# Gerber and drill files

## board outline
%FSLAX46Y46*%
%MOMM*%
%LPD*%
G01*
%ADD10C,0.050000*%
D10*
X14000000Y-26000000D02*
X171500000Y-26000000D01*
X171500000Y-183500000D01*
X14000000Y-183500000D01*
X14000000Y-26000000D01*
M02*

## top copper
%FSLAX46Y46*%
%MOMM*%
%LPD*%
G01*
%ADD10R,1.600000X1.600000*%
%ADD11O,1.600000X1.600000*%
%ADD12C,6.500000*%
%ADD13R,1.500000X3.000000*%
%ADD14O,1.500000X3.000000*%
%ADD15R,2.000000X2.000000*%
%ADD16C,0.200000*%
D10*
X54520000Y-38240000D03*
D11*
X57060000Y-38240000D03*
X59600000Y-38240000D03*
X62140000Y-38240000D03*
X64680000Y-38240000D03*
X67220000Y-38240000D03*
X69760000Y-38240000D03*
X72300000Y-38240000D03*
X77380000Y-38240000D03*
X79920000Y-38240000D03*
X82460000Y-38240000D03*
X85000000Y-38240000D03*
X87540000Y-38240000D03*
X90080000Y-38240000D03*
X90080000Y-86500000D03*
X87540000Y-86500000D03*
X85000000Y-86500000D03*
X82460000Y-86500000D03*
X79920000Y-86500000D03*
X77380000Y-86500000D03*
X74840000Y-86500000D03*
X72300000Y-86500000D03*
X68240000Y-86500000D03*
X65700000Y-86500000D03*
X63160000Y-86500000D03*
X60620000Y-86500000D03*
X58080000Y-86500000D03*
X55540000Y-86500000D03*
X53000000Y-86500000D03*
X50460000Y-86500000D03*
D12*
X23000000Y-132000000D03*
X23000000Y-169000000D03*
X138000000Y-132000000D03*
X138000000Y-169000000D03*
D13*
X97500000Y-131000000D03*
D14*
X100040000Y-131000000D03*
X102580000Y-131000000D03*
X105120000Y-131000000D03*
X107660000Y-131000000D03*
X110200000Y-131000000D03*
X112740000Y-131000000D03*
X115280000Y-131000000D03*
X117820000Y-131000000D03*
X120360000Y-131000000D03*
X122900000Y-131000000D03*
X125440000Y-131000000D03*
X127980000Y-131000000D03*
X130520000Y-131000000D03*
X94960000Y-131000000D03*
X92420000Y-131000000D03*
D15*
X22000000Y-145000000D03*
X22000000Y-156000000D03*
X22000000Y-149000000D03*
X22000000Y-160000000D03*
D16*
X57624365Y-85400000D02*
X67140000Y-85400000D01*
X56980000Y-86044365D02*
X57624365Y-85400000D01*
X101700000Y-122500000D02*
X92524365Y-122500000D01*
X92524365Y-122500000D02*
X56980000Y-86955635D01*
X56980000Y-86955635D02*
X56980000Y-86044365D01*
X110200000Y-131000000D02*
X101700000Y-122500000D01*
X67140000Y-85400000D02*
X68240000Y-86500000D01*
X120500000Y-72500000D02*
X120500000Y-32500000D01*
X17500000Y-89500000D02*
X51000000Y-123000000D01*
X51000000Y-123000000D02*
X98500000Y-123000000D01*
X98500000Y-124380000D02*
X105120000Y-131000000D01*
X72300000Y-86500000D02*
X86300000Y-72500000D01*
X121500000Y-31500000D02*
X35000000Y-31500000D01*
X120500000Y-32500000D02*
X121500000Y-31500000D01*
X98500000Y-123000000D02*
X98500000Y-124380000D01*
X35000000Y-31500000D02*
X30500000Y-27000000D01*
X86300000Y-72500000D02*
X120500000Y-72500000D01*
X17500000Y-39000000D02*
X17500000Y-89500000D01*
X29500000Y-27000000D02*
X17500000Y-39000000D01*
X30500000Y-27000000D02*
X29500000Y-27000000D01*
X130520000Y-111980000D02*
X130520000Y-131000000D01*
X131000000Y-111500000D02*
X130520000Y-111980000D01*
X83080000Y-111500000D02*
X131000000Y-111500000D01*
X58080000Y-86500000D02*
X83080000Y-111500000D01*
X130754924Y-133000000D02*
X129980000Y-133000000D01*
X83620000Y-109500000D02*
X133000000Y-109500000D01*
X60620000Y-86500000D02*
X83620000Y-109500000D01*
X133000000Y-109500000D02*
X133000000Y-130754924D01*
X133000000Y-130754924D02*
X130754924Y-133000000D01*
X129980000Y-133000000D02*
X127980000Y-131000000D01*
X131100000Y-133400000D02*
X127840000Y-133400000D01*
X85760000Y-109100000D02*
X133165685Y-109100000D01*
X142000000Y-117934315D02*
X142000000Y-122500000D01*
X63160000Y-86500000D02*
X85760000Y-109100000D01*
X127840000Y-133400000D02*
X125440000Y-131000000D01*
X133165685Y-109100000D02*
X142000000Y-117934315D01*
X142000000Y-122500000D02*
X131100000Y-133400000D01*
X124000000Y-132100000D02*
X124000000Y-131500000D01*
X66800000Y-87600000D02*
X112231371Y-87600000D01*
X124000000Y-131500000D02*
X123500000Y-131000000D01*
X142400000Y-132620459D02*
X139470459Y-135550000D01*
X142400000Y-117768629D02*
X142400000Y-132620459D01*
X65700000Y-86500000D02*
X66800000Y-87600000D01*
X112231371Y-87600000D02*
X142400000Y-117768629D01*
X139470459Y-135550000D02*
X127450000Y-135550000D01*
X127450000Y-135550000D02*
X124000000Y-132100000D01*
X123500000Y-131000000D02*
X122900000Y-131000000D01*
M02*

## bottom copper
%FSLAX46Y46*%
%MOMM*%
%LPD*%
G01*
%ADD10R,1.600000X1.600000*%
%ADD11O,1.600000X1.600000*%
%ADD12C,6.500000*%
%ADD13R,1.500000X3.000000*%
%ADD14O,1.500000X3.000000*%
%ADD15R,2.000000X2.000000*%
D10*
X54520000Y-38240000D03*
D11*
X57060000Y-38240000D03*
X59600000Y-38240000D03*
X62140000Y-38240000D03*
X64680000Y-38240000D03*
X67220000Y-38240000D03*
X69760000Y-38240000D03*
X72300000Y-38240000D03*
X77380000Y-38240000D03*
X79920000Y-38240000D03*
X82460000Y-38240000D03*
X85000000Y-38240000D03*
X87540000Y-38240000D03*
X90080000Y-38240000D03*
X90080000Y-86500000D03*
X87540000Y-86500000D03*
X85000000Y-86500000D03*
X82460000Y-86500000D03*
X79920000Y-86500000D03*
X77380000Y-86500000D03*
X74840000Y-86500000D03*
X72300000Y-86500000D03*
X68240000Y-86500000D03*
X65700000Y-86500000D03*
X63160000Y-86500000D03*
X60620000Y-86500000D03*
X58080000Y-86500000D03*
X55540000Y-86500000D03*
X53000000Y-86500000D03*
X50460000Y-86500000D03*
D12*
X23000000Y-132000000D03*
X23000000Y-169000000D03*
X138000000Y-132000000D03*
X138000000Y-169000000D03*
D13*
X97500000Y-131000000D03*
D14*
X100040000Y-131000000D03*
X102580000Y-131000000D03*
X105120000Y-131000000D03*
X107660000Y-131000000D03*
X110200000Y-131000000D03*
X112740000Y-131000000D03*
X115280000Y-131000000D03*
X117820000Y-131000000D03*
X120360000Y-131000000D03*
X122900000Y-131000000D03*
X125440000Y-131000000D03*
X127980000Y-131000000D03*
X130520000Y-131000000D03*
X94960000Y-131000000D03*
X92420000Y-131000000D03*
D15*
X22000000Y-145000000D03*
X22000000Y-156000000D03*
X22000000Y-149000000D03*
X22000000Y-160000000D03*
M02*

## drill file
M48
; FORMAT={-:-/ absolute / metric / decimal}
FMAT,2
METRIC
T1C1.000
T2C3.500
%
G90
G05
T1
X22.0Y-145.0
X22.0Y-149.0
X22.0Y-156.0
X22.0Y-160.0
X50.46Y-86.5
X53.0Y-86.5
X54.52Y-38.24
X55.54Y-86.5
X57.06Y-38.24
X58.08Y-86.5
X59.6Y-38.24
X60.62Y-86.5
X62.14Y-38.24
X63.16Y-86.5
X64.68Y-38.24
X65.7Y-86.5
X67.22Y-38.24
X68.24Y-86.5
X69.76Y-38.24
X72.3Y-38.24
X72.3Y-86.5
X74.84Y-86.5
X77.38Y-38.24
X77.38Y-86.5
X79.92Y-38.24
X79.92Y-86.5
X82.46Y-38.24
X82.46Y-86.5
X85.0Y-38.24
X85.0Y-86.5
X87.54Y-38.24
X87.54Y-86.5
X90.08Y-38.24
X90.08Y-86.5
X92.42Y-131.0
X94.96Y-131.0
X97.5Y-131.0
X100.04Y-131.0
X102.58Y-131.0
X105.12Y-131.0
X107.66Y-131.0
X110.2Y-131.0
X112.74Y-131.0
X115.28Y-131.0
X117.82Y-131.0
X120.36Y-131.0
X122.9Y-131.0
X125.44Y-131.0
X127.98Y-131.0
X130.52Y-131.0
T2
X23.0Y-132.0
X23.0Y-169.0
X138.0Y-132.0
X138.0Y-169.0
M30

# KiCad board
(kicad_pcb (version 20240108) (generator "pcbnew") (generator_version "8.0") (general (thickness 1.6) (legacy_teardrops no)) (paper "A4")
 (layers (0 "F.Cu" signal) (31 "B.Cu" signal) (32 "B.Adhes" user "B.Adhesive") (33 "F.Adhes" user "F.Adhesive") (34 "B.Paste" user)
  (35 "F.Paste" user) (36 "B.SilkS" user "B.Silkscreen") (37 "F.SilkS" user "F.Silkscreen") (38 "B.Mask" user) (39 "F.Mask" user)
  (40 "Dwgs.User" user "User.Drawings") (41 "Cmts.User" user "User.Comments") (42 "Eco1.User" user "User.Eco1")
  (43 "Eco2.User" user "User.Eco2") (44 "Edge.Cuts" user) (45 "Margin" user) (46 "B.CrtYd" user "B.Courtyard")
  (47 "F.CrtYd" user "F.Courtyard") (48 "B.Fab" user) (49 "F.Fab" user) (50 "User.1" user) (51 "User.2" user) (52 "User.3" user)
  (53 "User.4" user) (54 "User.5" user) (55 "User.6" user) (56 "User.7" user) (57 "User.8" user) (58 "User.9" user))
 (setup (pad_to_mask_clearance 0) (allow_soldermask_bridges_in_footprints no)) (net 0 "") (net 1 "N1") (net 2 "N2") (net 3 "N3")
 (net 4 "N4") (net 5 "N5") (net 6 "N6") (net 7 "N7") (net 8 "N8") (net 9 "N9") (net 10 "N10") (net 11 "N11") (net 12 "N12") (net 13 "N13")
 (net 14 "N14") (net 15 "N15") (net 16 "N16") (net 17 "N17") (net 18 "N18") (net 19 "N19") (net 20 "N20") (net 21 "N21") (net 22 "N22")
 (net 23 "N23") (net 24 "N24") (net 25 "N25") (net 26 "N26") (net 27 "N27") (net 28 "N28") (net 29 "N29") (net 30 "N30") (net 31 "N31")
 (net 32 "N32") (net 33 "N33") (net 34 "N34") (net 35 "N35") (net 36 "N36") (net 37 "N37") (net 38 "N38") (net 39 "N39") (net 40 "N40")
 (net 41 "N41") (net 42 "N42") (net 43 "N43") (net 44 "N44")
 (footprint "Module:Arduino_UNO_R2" (layer "F.Cu") (at 54.52 38.24)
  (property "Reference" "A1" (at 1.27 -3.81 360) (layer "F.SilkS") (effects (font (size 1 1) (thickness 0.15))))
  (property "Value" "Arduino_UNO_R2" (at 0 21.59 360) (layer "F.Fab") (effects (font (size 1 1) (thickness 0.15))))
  (pad "1" thru_hole rect (at 0 0 90) (size 1.6 1.6) (drill 1) (layers "*.Cu" "*.Mask") (remove_unused_layers no) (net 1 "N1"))
  (pad "2" thru_hole oval (at 2.54 0 90) (size 1.6 1.6) (drill 1) (layers "*.Cu" "*.Mask") (remove_unused_layers no) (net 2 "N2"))
  (pad "3" thru_hole oval (at 5.08 0 90) (size 1.6 1.6) (drill 1) (layers "*.Cu" "*.Mask") (remove_unused_layers no) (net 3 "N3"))
  (pad "4" thru_hole oval (at 7.62 0 90) (size 1.6 1.6) (drill 1) (layers "*.Cu" "*.Mask") (remove_unused_layers no) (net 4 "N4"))
  (pad "5" thru_hole oval (at 10.16 0 90) (size 1.6 1.6) (drill 1) (layers "*.Cu" "*.Mask") (remove_unused_layers no) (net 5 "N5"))
  (pad "6" thru_hole oval (at 12.7 0 90) (size 1.6 1.6) (drill 1) (layers "*.Cu" "*.Mask") (remove_unused_layers no) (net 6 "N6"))
  (pad "7" thru_hole oval (at 15.24 0 90) (size 1.6 1.6) (drill 1) (layers "*.Cu" "*.Mask") (remove_unused_layers no) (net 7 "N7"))
  (pad "8" thru_hole oval (at 17.78 0 90) (size 1.6 1.6) (drill 1) (layers "*.Cu" "*.Mask") (remove_unused_layers no) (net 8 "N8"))
  (pad "9" thru_hole oval (at 22.86 0 90) (size 1.6 1.6) (drill 1) (layers "*.Cu" "*.Mask") (remove_unused_layers no) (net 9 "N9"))
  (pad "10" thru_hole oval (at 25.4 0 90) (size 1.6 1.6) (drill 1) (layers "*.Cu" "*.Mask") (remove_unused_layers no) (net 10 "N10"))
  (pad "11" thru_hole oval (at 27.94 0 90) (size 1.6 1.6) (drill 1) (layers "*.Cu" "*.Mask") (remove_unused_layers no) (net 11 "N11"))
  (pad "12" thru_hole oval (at 30.48 0 90) (size 1.6 1.6) (drill 1) (layers "*.Cu" "*.Mask") (remove_unused_layers no) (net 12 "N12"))
  (pad "13" thru_hole oval (at 33.02 0 90) (size 1.6 1.6) (drill 1) (layers "*.Cu" "*.Mask") (remove_unused_layers no) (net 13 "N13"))
  (pad "14" thru_hole oval (at 35.56 0 90) (size 1.6 1.6) (drill 1) (layers "*.Cu" "*.Mask") (remove_unused_layers no) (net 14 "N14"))
  (pad "15" thru_hole oval (at 35.56 48.26 90) (size 1.6 1.6) (drill 1) (layers "*.Cu" "*.Mask") (remove_unused_layers no) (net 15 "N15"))
  (pad "16" thru_hole oval (at 33.02 48.26 90) (size 1.6 1.6) (drill 1) (layers "*.Cu" "*.Mask") (remove_unused_layers no) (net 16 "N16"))
  (pad "17" thru_hole oval (at 30.48 48.26 90) (size 1.6 1.6) (drill 1) (layers "*.Cu" "*.Mask") (remove_unused_layers no) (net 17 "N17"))
  (pad "18" thru_hole oval (at 27.94 48.26 90) (size 1.6 1.6) (drill 1) (layers "*.Cu" "*.Mask") (remove_unused_layers no) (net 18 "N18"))
  (pad "19" thru_hole oval (at 25.4 48.26 90) (size 1.6 1.6) (drill 1) (layers "*.Cu" "*.Mask") (remove_unused_layers no) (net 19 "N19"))
  (pad "20" thru_hole oval (at 22.86 48.26 90) (size 1.6 1.6) (drill 1) (layers "*.Cu" "*.Mask") (remove_unused_layers no) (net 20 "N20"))
  (pad "21" thru_hole oval (at 20.32 48.26 90) (size 1.6 1.6) (drill 1) (layers "*.Cu" "*.Mask") (remove_unused_layers no) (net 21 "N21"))
  (pad "22" thru_hole oval (at 17.78 48.26 90) (size 1.6 1.6) (drill 1) (layers "*.Cu" "*.Mask") (remove_unused_layers no) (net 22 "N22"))
  (pad "23" thru_hole oval (at 13.72 48.26 90) (size 1.6 1.6) (drill 1) (layers "*.Cu" "*.Mask") (remove_unused_layers no) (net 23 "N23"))
  (pad "24" thru_hole oval (at 11.18 48.26 90) (size 1.6 1.6) (drill 1) (layers "*.Cu" "*.Mask") (remove_unused_layers no) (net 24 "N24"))
  (pad "25" thru_hole oval (at 8.64 48.26 90) (size 1.6 1.6) (drill 1) (layers "*.Cu" "*.Mask") (remove_unused_layers no) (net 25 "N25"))
  (pad "26" thru_hole oval (at 6.1 48.26 90) (size 1.6 1.6) (drill 1) (layers "*.Cu" "*.Mask") (remove_unused_layers no) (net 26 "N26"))
  (pad "27" thru_hole oval (at 3.56 48.26 90) (size 1.6 1.6) (drill 1) (layers "*.Cu" "*.Mask") (remove_unused_layers no) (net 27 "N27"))
  (pad "28" thru_hole oval (at 1.02 48.26 90) (size 1.6 1.6) (drill 1) (layers "*.Cu" "*.Mask") (remove_unused_layers no) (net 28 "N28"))
  (pad "29" thru_hole oval (at -1.52 48.26 90) (size 1.6 1.6) (drill 1) (layers "*.Cu" "*.Mask") (remove_unused_layers no) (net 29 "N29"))
  (pad "30" thru_hole oval (at -4.06 48.26 90) (size 1.6 1.6) (drill 1) (layers "*.Cu" "*.Mask") (remove_unused_layers no) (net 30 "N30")))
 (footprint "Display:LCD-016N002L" (layer "F.Cu") (at 97.5 131)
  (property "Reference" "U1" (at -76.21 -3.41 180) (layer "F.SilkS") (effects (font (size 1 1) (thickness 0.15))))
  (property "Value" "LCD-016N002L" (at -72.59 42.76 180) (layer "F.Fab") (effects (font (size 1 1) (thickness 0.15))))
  (pad "" thru_hole circle (at -74.5 1 180) (size 6.5 6.5) (drill 3.5) (layers "*.Cu" "*.Mask") (remove_unused_layers no))
  (pad "" thru_hole circle (at -74.5 38 180) (size 6.5 6.5) (drill 3.5) (layers "*.Cu" "*.Mask") (remove_unused_layers no))
  (pad "" thru_hole circle (at 40.5 1 180) (size 6.5 6.5) (drill 3.5) (layers "*.Cu" "*.Mask") (remove_unused_layers no))
  (pad "" thru_hole circle (at 40.5 38 180) (size 6.5 6.5) (drill 3.5) (layers "*.Cu" "*.Mask") (remove_unused_layers no))
  (pad "1" thru_hole rect (at 0 0 180) (size 1.5 3) (drill 1) (layers "*.Cu" "*.Mask") (remove_unused_layers no) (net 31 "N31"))
  (pad "2" thru_hole oval (at 2.54 0 180) (size 1.5 3) (drill 1) (layers "*.Cu" "*.Mask") (remove_unused_layers no) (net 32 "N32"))
  (pad "3" thru_hole oval (at 5.08 0 180) (size 1.5 3) (drill 1) (layers "*.Cu" "*.Mask") (remove_unused_layers no) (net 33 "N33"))
  (pad "4" thru_hole oval (at 7.62 0 180) (size 1.5 3) (drill 1) (layers "*.Cu" "*.Mask") (remove_unused_layers no) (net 22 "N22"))
  (pad "5" thru_hole oval (at 10.16 0 180) (size 1.5 3) (drill 1) (layers "*.Cu" "*.Mask") (remove_unused_layers no) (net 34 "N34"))
  (pad "6" thru_hole oval (at 12.7 0 180) (size 1.5 3) (drill 1) (layers "*.Cu" "*.Mask") (remove_unused_layers no) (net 23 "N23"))
  (pad "7" thru_hole oval (at 15.24 0 180) (size 1.5 3) (drill 1) (layers "*.Cu" "*.Mask") (remove_unused_layers no) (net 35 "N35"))
  (pad "8" thru_hole oval (at 17.78 0 180) (size 1.5 3) (drill 1) (layers "*.Cu" "*.Mask") (remove_unused_layers no) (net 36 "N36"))
  (pad "9" thru_hole oval (at 20.32 0 180) (size 1.5 3) (drill 1) (layers "*.Cu" "*.Mask") (remove_unused_layers no) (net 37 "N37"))
  (pad "10" thru_hole oval (at 22.86 0 180) (size 1.5 3) (drill 1) (layers "*.Cu" "*.Mask") (remove_unused_layers no) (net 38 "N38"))
  (pad "11" thru_hole oval (at 25.4 0 180) (size 1.5 3) (drill 1) (layers "*.Cu" "*.Mask") (remove_unused_layers no) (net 24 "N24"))
  (pad "12" thru_hole oval (at 27.94 0 180) (size 1.5 3) (drill 1) (layers "*.Cu" "*.Mask") (remove_unused_layers no) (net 25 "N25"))
  (pad "13" thru_hole oval (at 30.48 0 180) (size 1.5 3) (drill 1) (layers "*.Cu" "*.Mask") (remove_unused_layers no) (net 26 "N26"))
  (pad "14" thru_hole oval (at 33.02 0 180) (size 1.5 3) (drill 1) (layers "*.Cu" "*.Mask") (remove_unused_layers no) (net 27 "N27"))
  (pad "15" thru_hole oval (at -2.54 0 180) (size 1.5 3) (drill 1) (layers "*.Cu" "*.Mask") (remove_unused_layers no) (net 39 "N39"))
  (pad "16" thru_hole oval (at -5.08 0 180) (size 1.5 3) (drill 1) (layers "*.Cu" "*.Mask") (remove_unused_layers no) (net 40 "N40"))
  (pad "A1" thru_hole rect (at -75.5 14 180) (size 2 2) (drill 1) (layers "*.Cu" "*.Mask") (remove_unused_layers no) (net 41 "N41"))
  (pad "A2" thru_hole rect (at -75.5 25 180) (size 2 2) (drill 1) (layers "*.Cu" "*.Mask") (remove_unused_layers no) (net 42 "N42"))
  (pad "K1" thru_hole rect (at -75.5 18 180) (size 2 2) (drill 1) (layers "*.Cu" "*.Mask") (remove_unused_layers no) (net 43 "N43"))
  (pad "K2" thru_hole rect (at -75.5 29 180) (size 2 2) (drill 1) (layers "*.Cu" "*.Mask") (remove_unused_layers no) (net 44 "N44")))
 (gr_rect (start 14 26) (end 171.5 183.5) (stroke (width 0.05) (type default)) (fill none) (layer "Edge.Cuts"))
 (segment (start 57.624365 85.4) (end 67.14 85.4) (width 0.2) (layer "F.Cu") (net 23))
 (segment (start 56.98 86.044365) (end 57.624365 85.4) (width 0.2) (layer "F.Cu") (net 23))
 (segment (start 101.7 122.5) (end 92.524365 122.5) (width 0.2) (layer "F.Cu") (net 23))
 (segment (start 92.524365 122.5) (end 56.98 86.955635) (width 0.2) (layer "F.Cu") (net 23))
 (segment (start 56.98 86.955635) (end 56.98 86.044365) (width 0.2) (layer "F.Cu") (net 23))
 (segment (start 110.2 131) (end 101.7 122.5) (width 0.2) (layer "F.Cu") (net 23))
 (segment (start 67.14 85.4) (end 68.24 86.5) (width 0.2) (layer "F.Cu") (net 23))
 (segment (start 120.5 72.5) (end 120.5 32.5) (width 0.2) (layer "F.Cu") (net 22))
 (segment (start 17.5 89.5) (end 51 123) (width 0.2) (layer "F.Cu") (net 22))
 (segment (start 51 123) (end 98.5 123) (width 0.2) (layer "F.Cu") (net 22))
 (segment (start 98.5 124.38) (end 105.12 131) (width 0.2) (layer "F.Cu") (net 22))
 (segment (start 72.3 86.5) (end 86.3 72.5) (width 0.2) (layer "F.Cu") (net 22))
 (segment (start 121.5 31.5) (end 35 31.5) (width 0.2) (layer "F.Cu") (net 22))
 (segment (start 120.5 32.5) (end 121.5 31.5) (width 0.2) (layer "F.Cu") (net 22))
 (segment (start 98.5 123) (end 98.5 124.38) (width 0.2) (layer "F.Cu") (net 22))
 (segment (start 35 31.5) (end 30.5 27) (width 0.2) (layer "F.Cu") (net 22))
 (segment (start 86.3 72.5) (end 120.5 72.5) (width 0.2) (layer "F.Cu") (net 22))
 (segment (start 17.5 39) (end 17.5 89.5) (width 0.2) (layer "F.Cu") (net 22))
 (segment (start 29.5 27) (end 17.5 39) (width 0.2) (layer "F.Cu") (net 22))
 (segment (start 30.5 27) (end 29.5 27) (width 0.2) (layer "F.Cu") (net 22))
 (segment (start 130.52 111.98) (end 130.52 131) (width 0.2) (layer "F.Cu") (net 27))
 (segment (start 131 111.5) (end 130.52 111.98) (width 0.2) (layer "F.Cu") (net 27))
 (segment (start 83.08 111.5) (end 131 111.5) (width 0.2) (layer "F.Cu") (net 27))
 (segment (start 58.08 86.5) (end 83.08 111.5) (width 0.2) (layer "F.Cu") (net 27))
 (segment (start 130.754924 133) (end 129.98 133) (width 0.2) (layer "F.Cu") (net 26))
 (segment (start 83.62 109.5) (end 133 109.5) (width 0.2) (layer "F.Cu") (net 26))
 (segment (start 60.62 86.5) (end 83.62 109.5) (width 0.2) (layer "F.Cu") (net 26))
 (segment (start 133 109.5) (end 133 130.754924) (width 0.2) (layer "F.Cu") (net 26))
 (segment (start 133 130.754924) (end 130.754924 133) (width 0.2) (layer "F.Cu") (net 26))
 (segment (start 129.98 133) (end 127.98 131) (width 0.2) (layer "F.Cu") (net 26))
 (segment (start 131.1 133.4) (end 127.84 133.4) (width 0.2) (layer "F.Cu") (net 25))
 (segment (start 85.76 109.1) (end 133.165685 109.1) (width 0.2) (layer "F.Cu") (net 25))
 (segment (start 142 117.934315) (end 142 122.5) (width 0.2) (layer "F.Cu") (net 25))
 (segment (start 63.16 86.5) (end 85.76 109.1) (width 0.2) (layer "F.Cu") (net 25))
 (segment (start 127.84 133.4) (end 125.44 131) (width 0.2) (layer "F.Cu") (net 25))
 (segment (start 133.165685 109.1) (end 142 117.934315) (width 0.2) (layer "F.Cu") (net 25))
 (segment (start 142 122.5) (end 131.1 133.4) (width 0.2) (layer "F.Cu") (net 25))
 (segment (start 124 132.1) (end 124 131.5) (width 0.2) (layer "F.Cu") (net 24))
 (segment (start 66.8 87.6) (end 112.231371 87.6) (width 0.2) (layer "F.Cu") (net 24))
 (segment (start 124 131.5) (end 123.5 131) (width 0.2) (layer "F.Cu") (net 24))
 (segment (start 142.4 132.620459) (end 139.470459 135.55) (width 0.2) (layer "F.Cu") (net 24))
 (segment (start 142.4 117.768629) (end 142.4 132.620459) (width 0.2) (layer "F.Cu") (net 24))
 (segment (start 65.7 86.5) (end 66.8 87.6) (width 0.2) (layer "F.Cu") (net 24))
 (segment (start 112.231371 87.6) (end 142.4 117.768629) (width 0.2) (layer "F.Cu") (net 24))
 (segment (start 139.470459 135.55) (end 127.45 135.55) (width 0.2) (layer "F.Cu") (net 24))
 (segment (start 127.45 135.55) (end 124 132.1) (width 0.2) (layer "F.Cu") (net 24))
 (segment (start 123.5 131) (end 122.9 131) (width 0.2) (layer "F.Cu") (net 24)))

